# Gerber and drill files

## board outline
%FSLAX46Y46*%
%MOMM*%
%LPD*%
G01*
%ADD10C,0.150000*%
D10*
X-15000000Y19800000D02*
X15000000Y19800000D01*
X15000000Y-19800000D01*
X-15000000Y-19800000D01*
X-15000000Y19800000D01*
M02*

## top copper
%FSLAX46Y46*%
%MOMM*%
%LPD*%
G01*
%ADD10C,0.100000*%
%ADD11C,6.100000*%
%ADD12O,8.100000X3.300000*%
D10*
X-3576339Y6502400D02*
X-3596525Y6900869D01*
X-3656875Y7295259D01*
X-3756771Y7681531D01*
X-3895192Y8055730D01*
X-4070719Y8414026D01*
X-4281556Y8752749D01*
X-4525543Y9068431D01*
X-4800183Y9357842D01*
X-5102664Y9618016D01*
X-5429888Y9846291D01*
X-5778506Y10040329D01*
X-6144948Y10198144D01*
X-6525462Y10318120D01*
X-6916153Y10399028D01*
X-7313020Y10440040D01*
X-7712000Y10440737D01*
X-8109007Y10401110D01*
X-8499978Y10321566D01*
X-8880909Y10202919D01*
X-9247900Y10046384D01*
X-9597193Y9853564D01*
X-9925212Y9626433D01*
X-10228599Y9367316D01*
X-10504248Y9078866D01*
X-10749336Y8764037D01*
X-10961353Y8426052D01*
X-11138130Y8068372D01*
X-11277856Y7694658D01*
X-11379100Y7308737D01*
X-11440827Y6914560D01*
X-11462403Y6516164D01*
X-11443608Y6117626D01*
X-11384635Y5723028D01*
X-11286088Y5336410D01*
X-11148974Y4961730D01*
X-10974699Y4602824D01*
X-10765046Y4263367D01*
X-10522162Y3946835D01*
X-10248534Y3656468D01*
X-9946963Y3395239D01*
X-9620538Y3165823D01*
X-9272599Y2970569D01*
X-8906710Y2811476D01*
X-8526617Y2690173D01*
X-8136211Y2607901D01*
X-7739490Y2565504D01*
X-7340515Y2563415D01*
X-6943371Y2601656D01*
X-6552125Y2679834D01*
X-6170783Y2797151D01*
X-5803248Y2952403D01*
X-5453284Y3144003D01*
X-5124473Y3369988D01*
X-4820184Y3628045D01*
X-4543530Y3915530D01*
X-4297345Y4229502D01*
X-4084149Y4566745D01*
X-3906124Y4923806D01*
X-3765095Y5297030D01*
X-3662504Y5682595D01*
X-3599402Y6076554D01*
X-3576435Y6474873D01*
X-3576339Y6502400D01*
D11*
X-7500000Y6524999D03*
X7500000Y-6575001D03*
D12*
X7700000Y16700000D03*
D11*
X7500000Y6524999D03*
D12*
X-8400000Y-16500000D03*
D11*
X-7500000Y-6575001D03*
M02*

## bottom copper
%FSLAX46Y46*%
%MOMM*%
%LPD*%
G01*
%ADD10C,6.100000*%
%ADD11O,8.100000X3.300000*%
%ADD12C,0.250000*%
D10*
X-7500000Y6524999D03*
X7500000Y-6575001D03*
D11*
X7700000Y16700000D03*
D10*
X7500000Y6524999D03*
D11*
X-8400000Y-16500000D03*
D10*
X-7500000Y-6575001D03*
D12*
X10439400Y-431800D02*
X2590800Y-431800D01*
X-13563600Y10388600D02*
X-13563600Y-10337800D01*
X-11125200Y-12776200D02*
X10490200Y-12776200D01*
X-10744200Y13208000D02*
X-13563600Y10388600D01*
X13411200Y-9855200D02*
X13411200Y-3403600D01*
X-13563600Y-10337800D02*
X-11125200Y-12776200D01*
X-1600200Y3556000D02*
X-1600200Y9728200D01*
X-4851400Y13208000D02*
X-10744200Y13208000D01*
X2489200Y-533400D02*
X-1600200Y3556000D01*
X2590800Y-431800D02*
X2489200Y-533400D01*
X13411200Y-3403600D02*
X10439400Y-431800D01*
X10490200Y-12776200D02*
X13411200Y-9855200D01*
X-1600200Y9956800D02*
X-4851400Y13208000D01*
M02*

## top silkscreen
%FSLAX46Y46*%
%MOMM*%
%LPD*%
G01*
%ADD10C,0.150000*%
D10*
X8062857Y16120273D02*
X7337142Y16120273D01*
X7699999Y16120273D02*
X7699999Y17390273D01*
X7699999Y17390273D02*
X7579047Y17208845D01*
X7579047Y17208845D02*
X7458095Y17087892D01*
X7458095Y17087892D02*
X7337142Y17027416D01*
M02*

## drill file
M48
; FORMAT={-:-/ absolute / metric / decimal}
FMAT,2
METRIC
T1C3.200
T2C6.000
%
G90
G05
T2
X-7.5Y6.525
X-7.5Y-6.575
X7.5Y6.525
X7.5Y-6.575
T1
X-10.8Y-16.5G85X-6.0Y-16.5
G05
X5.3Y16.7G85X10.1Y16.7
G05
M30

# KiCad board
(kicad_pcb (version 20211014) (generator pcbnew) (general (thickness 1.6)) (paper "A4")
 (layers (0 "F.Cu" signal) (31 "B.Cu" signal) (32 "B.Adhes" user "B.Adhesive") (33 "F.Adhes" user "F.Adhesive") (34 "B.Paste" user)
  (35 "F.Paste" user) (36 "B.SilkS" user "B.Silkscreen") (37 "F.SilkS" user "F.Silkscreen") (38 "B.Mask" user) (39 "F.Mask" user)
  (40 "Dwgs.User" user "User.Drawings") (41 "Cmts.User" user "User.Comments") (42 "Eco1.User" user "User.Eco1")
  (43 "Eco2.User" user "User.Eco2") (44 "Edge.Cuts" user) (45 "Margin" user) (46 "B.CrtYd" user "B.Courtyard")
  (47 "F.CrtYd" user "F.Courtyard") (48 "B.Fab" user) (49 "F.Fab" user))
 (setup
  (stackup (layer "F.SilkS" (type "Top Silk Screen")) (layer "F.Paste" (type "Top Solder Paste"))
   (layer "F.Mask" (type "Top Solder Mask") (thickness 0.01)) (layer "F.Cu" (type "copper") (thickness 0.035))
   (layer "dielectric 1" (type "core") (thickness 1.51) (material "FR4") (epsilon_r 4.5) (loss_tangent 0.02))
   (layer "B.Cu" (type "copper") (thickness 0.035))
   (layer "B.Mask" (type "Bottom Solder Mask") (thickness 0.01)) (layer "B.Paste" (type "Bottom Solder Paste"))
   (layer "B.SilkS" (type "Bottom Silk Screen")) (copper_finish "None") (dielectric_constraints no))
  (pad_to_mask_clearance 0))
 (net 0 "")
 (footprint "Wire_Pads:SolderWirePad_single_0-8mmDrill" (layer "F.Cu") (at -7.5 -6.524999)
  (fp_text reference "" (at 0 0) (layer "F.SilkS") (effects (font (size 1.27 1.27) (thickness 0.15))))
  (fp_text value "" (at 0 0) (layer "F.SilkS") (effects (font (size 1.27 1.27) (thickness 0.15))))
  (pad "1" thru_hole circle locked (at 0 0) (size 6.1 6.1) (drill 6) (layers *.Cu *.Mask)))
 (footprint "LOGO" (layer "F.Cu") (at 0 0)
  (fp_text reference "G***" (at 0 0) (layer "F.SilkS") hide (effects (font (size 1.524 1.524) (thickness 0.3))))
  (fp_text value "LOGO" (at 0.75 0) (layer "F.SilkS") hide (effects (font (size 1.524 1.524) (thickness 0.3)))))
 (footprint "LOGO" (layer "F.Cu") (at 0 0)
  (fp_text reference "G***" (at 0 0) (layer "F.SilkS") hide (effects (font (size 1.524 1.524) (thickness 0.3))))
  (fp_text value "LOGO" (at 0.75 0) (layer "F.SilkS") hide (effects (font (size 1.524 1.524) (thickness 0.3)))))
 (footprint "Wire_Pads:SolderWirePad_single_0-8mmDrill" (layer "F.Cu") (at 7.5 6.575001)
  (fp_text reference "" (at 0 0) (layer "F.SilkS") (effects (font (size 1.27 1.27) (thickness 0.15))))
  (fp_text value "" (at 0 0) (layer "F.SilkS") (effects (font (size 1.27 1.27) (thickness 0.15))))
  (pad "4" thru_hole circle locked (at 0 0) (size 6.1 6.1) (drill 6) (layers *.Cu *.Mask)))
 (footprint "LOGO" (layer "F.Cu") (at 0 0)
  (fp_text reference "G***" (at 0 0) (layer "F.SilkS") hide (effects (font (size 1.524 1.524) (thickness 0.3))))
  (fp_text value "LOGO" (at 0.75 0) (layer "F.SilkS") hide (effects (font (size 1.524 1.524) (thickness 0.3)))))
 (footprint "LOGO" (layer "F.Cu") (at 0 0)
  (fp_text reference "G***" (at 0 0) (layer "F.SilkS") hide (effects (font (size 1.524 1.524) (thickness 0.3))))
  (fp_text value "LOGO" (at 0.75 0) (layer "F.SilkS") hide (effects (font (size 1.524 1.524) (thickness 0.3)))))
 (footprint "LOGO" (layer "F.Cu") (at 0.591786 0.539509)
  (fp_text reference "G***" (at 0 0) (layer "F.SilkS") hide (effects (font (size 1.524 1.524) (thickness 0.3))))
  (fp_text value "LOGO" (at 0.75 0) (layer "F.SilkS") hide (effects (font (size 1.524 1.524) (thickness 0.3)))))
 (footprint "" (layer "F.Cu") (at 7.7 -16.7)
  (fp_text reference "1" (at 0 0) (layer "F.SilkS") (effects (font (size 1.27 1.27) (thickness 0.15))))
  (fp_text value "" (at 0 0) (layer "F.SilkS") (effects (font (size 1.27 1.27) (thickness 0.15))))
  (pad "2" thru_hole oval locked (at 0 0) (size 8.1 3.3) (drill oval 8 3.2) (layers *.Cu *.Mask)))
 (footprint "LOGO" (layer "F.Cu") (at 0 0)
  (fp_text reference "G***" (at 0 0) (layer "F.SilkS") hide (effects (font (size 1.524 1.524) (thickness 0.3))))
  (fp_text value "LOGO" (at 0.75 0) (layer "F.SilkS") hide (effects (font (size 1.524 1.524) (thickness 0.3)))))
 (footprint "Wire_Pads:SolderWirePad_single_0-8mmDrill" (layer "F.Cu") (at 7.5 -6.524999)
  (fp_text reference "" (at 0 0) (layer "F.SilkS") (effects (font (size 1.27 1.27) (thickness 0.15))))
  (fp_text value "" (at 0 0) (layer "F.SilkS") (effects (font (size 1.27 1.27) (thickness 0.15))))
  (pad "2" thru_hole circle locked (at 0 0) (size 6.1 6.1) (drill 6) (layers *.Cu *.Mask)))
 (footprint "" (layer "F.Cu") (at -8.4 16.5)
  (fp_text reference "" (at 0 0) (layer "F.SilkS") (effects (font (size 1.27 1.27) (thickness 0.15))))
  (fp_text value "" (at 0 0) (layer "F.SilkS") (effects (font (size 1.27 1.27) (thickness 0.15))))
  (pad "2" thru_hole oval locked (at 0 0) (size 8.1 3.3) (drill oval 8 3.2) (layers *.Cu *.Mask)))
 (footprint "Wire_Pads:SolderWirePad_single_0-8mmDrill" (layer "F.Cu") (at -7.5 6.575001)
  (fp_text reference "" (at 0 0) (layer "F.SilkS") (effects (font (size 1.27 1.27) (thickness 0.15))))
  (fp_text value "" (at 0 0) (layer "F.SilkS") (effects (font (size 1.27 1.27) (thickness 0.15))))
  (pad "3" thru_hole circle locked (at 0 0) (size 6.1 6.1) (drill 6) (layers *.Cu *.Mask)))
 (gr_poly
  (pts (xy -3.576339 -6.5024) (xy -3.596525 -6.900869) (xy -3.656875 -7.295259) (xy -3.756771 -7.681531) (xy -3.895192 -8.05573)
   (xy -4.070719 -8.414026) (xy -4.281556 -8.752749) (xy -4.525543 -9.068431) (xy -4.800183 -9.357842) (xy -5.102664 -9.618016)
   (xy -5.429888 -9.846291) (xy -5.778506 -10.040329) (xy -6.144948 -10.198144) (xy -6.525462 -10.31812) (xy -6.916153 -10.399028)
   (xy -7.31302 -10.44004) (xy -7.712 -10.440737) (xy -8.109007 -10.40111) (xy -8.499978 -10.321566) (xy -8.880909 -10.202919)
   (xy -9.2479 -10.046384) (xy -9.597193 -9.853564) (xy -9.925212 -9.626433) (xy -10.228599 -9.367316) (xy -10.504248 -9.078866)
   (xy -10.749336 -8.764037) (xy -10.961353 -8.426052) (xy -11.13813 -8.068372) (xy -11.277856 -7.694658) (xy -11.3791 -7.308737)
   (xy -11.440827 -6.91456) (xy -11.462403 -6.516164) (xy -11.443608 -6.117626) (xy -11.384635 -5.723028) (xy -11.286088 -5.33641)
   (xy -11.148974 -4.96173) (xy -10.974699 -4.602824) (xy -10.765046 -4.263367) (xy -10.522162 -3.946835) (xy -10.248534 -3.656468)
   (xy -9.946963 -3.395239) (xy -9.620538 -3.165823) (xy -9.272599 -2.970569) (xy -8.90671 -2.811476) (xy -8.526617 -2.690173)
   (xy -8.136211 -2.607901) (xy -7.73949 -2.565504) (xy -7.340515 -2.563415) (xy -6.943371 -2.601656) (xy -6.552125 -2.679834)
   (xy -6.170783 -2.797151) (xy -5.803248 -2.952403) (xy -5.453284 -3.144003) (xy -5.124473 -3.369988) (xy -4.820184 -3.628045)
   (xy -4.54353 -3.91553) (xy -4.297345 -4.229502) (xy -4.084149 -4.566745) (xy -3.906124 -4.923806) (xy -3.765095 -5.29703)
   (xy -3.662504 -5.682595) (xy -3.599402 -6.076554) (xy -3.576435 -6.474873))
  (layer "F.Cu") (width 0.1) (fill none))
 (gr_rect (start -15 -19.8) (end 15 19.8) (layer "Edge.Cuts") (width 0.15) (fill none))
 (segment (start 10.4394 0.4318) (end 2.5908 0.4318) (width 0.25) (layer "B.Cu") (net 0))
 (segment (start -13.5636 -10.3886) (end -13.5636 10.3378) (width 0.25) (layer "B.Cu") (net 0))
 (segment (start -11.1252 12.7762) (end 10.4902 12.7762) (width 0.25) (layer "B.Cu") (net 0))
 (segment (start -10.7442 -13.208) (end -13.5636 -10.3886) (width 0.25) (layer "B.Cu") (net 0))
 (segment (start 13.4112 9.8552) (end 13.4112 3.4036) (width 0.25) (layer "B.Cu") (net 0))
 (segment (start -13.5636 10.3378) (end -11.1252 12.7762) (width 0.25) (layer "B.Cu") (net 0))
 (segment (start -1.6002 -3.556) (end -1.6002 -9.7282) (width 0.25) (layer "B.Cu") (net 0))
 (segment (start -4.8514 -13.208) (end -10.7442 -13.208) (width 0.25) (layer "B.Cu") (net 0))
 (segment (start 2.4892 0.5334) (end -1.6002 -3.556) (width 0.25) (layer "B.Cu") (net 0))
 (segment (start 2.5908 0.4318) (end 2.4892 0.5334) (width 0.25) (layer "B.Cu") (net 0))
 (segment (start 13.4112 3.4036) (end 10.4394 0.4318) (width 0.25) (layer "B.Cu") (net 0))
 (segment (start 10.4902 12.7762) (end 13.4112 9.8552) (width 0.25) (layer "B.Cu") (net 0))
 (segment (start -1.6002 -9.9568) (end -4.8514 -13.208) (width 0.25) (layer "B.Cu") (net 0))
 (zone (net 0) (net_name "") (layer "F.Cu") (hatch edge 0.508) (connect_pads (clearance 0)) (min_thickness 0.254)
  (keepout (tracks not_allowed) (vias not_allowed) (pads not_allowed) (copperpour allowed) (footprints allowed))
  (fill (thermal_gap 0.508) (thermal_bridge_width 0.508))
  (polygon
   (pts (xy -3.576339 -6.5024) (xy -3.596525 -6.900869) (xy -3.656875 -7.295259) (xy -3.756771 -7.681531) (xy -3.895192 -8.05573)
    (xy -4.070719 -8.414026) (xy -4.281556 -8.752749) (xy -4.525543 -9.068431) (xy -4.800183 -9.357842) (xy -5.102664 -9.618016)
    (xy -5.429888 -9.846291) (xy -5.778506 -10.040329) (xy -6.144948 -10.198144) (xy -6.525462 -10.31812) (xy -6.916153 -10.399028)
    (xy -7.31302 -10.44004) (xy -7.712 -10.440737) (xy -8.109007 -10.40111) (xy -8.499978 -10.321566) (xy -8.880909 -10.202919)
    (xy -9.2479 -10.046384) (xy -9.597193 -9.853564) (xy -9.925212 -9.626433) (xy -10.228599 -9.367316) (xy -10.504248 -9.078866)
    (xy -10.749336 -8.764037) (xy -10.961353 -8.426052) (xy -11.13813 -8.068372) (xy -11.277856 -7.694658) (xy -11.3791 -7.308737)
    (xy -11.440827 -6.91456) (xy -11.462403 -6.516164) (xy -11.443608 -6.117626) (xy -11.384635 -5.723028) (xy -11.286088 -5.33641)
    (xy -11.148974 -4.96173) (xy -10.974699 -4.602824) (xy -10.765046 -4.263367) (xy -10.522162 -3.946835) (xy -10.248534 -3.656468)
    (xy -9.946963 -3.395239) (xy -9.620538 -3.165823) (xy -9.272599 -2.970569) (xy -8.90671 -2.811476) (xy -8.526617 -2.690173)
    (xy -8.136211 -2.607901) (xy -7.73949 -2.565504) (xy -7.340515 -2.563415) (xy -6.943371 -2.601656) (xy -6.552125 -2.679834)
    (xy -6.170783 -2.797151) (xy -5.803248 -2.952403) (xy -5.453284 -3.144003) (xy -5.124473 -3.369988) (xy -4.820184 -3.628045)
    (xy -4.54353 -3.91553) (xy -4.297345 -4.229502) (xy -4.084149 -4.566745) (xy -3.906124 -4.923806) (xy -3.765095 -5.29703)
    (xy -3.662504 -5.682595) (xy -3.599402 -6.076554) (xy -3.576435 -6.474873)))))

